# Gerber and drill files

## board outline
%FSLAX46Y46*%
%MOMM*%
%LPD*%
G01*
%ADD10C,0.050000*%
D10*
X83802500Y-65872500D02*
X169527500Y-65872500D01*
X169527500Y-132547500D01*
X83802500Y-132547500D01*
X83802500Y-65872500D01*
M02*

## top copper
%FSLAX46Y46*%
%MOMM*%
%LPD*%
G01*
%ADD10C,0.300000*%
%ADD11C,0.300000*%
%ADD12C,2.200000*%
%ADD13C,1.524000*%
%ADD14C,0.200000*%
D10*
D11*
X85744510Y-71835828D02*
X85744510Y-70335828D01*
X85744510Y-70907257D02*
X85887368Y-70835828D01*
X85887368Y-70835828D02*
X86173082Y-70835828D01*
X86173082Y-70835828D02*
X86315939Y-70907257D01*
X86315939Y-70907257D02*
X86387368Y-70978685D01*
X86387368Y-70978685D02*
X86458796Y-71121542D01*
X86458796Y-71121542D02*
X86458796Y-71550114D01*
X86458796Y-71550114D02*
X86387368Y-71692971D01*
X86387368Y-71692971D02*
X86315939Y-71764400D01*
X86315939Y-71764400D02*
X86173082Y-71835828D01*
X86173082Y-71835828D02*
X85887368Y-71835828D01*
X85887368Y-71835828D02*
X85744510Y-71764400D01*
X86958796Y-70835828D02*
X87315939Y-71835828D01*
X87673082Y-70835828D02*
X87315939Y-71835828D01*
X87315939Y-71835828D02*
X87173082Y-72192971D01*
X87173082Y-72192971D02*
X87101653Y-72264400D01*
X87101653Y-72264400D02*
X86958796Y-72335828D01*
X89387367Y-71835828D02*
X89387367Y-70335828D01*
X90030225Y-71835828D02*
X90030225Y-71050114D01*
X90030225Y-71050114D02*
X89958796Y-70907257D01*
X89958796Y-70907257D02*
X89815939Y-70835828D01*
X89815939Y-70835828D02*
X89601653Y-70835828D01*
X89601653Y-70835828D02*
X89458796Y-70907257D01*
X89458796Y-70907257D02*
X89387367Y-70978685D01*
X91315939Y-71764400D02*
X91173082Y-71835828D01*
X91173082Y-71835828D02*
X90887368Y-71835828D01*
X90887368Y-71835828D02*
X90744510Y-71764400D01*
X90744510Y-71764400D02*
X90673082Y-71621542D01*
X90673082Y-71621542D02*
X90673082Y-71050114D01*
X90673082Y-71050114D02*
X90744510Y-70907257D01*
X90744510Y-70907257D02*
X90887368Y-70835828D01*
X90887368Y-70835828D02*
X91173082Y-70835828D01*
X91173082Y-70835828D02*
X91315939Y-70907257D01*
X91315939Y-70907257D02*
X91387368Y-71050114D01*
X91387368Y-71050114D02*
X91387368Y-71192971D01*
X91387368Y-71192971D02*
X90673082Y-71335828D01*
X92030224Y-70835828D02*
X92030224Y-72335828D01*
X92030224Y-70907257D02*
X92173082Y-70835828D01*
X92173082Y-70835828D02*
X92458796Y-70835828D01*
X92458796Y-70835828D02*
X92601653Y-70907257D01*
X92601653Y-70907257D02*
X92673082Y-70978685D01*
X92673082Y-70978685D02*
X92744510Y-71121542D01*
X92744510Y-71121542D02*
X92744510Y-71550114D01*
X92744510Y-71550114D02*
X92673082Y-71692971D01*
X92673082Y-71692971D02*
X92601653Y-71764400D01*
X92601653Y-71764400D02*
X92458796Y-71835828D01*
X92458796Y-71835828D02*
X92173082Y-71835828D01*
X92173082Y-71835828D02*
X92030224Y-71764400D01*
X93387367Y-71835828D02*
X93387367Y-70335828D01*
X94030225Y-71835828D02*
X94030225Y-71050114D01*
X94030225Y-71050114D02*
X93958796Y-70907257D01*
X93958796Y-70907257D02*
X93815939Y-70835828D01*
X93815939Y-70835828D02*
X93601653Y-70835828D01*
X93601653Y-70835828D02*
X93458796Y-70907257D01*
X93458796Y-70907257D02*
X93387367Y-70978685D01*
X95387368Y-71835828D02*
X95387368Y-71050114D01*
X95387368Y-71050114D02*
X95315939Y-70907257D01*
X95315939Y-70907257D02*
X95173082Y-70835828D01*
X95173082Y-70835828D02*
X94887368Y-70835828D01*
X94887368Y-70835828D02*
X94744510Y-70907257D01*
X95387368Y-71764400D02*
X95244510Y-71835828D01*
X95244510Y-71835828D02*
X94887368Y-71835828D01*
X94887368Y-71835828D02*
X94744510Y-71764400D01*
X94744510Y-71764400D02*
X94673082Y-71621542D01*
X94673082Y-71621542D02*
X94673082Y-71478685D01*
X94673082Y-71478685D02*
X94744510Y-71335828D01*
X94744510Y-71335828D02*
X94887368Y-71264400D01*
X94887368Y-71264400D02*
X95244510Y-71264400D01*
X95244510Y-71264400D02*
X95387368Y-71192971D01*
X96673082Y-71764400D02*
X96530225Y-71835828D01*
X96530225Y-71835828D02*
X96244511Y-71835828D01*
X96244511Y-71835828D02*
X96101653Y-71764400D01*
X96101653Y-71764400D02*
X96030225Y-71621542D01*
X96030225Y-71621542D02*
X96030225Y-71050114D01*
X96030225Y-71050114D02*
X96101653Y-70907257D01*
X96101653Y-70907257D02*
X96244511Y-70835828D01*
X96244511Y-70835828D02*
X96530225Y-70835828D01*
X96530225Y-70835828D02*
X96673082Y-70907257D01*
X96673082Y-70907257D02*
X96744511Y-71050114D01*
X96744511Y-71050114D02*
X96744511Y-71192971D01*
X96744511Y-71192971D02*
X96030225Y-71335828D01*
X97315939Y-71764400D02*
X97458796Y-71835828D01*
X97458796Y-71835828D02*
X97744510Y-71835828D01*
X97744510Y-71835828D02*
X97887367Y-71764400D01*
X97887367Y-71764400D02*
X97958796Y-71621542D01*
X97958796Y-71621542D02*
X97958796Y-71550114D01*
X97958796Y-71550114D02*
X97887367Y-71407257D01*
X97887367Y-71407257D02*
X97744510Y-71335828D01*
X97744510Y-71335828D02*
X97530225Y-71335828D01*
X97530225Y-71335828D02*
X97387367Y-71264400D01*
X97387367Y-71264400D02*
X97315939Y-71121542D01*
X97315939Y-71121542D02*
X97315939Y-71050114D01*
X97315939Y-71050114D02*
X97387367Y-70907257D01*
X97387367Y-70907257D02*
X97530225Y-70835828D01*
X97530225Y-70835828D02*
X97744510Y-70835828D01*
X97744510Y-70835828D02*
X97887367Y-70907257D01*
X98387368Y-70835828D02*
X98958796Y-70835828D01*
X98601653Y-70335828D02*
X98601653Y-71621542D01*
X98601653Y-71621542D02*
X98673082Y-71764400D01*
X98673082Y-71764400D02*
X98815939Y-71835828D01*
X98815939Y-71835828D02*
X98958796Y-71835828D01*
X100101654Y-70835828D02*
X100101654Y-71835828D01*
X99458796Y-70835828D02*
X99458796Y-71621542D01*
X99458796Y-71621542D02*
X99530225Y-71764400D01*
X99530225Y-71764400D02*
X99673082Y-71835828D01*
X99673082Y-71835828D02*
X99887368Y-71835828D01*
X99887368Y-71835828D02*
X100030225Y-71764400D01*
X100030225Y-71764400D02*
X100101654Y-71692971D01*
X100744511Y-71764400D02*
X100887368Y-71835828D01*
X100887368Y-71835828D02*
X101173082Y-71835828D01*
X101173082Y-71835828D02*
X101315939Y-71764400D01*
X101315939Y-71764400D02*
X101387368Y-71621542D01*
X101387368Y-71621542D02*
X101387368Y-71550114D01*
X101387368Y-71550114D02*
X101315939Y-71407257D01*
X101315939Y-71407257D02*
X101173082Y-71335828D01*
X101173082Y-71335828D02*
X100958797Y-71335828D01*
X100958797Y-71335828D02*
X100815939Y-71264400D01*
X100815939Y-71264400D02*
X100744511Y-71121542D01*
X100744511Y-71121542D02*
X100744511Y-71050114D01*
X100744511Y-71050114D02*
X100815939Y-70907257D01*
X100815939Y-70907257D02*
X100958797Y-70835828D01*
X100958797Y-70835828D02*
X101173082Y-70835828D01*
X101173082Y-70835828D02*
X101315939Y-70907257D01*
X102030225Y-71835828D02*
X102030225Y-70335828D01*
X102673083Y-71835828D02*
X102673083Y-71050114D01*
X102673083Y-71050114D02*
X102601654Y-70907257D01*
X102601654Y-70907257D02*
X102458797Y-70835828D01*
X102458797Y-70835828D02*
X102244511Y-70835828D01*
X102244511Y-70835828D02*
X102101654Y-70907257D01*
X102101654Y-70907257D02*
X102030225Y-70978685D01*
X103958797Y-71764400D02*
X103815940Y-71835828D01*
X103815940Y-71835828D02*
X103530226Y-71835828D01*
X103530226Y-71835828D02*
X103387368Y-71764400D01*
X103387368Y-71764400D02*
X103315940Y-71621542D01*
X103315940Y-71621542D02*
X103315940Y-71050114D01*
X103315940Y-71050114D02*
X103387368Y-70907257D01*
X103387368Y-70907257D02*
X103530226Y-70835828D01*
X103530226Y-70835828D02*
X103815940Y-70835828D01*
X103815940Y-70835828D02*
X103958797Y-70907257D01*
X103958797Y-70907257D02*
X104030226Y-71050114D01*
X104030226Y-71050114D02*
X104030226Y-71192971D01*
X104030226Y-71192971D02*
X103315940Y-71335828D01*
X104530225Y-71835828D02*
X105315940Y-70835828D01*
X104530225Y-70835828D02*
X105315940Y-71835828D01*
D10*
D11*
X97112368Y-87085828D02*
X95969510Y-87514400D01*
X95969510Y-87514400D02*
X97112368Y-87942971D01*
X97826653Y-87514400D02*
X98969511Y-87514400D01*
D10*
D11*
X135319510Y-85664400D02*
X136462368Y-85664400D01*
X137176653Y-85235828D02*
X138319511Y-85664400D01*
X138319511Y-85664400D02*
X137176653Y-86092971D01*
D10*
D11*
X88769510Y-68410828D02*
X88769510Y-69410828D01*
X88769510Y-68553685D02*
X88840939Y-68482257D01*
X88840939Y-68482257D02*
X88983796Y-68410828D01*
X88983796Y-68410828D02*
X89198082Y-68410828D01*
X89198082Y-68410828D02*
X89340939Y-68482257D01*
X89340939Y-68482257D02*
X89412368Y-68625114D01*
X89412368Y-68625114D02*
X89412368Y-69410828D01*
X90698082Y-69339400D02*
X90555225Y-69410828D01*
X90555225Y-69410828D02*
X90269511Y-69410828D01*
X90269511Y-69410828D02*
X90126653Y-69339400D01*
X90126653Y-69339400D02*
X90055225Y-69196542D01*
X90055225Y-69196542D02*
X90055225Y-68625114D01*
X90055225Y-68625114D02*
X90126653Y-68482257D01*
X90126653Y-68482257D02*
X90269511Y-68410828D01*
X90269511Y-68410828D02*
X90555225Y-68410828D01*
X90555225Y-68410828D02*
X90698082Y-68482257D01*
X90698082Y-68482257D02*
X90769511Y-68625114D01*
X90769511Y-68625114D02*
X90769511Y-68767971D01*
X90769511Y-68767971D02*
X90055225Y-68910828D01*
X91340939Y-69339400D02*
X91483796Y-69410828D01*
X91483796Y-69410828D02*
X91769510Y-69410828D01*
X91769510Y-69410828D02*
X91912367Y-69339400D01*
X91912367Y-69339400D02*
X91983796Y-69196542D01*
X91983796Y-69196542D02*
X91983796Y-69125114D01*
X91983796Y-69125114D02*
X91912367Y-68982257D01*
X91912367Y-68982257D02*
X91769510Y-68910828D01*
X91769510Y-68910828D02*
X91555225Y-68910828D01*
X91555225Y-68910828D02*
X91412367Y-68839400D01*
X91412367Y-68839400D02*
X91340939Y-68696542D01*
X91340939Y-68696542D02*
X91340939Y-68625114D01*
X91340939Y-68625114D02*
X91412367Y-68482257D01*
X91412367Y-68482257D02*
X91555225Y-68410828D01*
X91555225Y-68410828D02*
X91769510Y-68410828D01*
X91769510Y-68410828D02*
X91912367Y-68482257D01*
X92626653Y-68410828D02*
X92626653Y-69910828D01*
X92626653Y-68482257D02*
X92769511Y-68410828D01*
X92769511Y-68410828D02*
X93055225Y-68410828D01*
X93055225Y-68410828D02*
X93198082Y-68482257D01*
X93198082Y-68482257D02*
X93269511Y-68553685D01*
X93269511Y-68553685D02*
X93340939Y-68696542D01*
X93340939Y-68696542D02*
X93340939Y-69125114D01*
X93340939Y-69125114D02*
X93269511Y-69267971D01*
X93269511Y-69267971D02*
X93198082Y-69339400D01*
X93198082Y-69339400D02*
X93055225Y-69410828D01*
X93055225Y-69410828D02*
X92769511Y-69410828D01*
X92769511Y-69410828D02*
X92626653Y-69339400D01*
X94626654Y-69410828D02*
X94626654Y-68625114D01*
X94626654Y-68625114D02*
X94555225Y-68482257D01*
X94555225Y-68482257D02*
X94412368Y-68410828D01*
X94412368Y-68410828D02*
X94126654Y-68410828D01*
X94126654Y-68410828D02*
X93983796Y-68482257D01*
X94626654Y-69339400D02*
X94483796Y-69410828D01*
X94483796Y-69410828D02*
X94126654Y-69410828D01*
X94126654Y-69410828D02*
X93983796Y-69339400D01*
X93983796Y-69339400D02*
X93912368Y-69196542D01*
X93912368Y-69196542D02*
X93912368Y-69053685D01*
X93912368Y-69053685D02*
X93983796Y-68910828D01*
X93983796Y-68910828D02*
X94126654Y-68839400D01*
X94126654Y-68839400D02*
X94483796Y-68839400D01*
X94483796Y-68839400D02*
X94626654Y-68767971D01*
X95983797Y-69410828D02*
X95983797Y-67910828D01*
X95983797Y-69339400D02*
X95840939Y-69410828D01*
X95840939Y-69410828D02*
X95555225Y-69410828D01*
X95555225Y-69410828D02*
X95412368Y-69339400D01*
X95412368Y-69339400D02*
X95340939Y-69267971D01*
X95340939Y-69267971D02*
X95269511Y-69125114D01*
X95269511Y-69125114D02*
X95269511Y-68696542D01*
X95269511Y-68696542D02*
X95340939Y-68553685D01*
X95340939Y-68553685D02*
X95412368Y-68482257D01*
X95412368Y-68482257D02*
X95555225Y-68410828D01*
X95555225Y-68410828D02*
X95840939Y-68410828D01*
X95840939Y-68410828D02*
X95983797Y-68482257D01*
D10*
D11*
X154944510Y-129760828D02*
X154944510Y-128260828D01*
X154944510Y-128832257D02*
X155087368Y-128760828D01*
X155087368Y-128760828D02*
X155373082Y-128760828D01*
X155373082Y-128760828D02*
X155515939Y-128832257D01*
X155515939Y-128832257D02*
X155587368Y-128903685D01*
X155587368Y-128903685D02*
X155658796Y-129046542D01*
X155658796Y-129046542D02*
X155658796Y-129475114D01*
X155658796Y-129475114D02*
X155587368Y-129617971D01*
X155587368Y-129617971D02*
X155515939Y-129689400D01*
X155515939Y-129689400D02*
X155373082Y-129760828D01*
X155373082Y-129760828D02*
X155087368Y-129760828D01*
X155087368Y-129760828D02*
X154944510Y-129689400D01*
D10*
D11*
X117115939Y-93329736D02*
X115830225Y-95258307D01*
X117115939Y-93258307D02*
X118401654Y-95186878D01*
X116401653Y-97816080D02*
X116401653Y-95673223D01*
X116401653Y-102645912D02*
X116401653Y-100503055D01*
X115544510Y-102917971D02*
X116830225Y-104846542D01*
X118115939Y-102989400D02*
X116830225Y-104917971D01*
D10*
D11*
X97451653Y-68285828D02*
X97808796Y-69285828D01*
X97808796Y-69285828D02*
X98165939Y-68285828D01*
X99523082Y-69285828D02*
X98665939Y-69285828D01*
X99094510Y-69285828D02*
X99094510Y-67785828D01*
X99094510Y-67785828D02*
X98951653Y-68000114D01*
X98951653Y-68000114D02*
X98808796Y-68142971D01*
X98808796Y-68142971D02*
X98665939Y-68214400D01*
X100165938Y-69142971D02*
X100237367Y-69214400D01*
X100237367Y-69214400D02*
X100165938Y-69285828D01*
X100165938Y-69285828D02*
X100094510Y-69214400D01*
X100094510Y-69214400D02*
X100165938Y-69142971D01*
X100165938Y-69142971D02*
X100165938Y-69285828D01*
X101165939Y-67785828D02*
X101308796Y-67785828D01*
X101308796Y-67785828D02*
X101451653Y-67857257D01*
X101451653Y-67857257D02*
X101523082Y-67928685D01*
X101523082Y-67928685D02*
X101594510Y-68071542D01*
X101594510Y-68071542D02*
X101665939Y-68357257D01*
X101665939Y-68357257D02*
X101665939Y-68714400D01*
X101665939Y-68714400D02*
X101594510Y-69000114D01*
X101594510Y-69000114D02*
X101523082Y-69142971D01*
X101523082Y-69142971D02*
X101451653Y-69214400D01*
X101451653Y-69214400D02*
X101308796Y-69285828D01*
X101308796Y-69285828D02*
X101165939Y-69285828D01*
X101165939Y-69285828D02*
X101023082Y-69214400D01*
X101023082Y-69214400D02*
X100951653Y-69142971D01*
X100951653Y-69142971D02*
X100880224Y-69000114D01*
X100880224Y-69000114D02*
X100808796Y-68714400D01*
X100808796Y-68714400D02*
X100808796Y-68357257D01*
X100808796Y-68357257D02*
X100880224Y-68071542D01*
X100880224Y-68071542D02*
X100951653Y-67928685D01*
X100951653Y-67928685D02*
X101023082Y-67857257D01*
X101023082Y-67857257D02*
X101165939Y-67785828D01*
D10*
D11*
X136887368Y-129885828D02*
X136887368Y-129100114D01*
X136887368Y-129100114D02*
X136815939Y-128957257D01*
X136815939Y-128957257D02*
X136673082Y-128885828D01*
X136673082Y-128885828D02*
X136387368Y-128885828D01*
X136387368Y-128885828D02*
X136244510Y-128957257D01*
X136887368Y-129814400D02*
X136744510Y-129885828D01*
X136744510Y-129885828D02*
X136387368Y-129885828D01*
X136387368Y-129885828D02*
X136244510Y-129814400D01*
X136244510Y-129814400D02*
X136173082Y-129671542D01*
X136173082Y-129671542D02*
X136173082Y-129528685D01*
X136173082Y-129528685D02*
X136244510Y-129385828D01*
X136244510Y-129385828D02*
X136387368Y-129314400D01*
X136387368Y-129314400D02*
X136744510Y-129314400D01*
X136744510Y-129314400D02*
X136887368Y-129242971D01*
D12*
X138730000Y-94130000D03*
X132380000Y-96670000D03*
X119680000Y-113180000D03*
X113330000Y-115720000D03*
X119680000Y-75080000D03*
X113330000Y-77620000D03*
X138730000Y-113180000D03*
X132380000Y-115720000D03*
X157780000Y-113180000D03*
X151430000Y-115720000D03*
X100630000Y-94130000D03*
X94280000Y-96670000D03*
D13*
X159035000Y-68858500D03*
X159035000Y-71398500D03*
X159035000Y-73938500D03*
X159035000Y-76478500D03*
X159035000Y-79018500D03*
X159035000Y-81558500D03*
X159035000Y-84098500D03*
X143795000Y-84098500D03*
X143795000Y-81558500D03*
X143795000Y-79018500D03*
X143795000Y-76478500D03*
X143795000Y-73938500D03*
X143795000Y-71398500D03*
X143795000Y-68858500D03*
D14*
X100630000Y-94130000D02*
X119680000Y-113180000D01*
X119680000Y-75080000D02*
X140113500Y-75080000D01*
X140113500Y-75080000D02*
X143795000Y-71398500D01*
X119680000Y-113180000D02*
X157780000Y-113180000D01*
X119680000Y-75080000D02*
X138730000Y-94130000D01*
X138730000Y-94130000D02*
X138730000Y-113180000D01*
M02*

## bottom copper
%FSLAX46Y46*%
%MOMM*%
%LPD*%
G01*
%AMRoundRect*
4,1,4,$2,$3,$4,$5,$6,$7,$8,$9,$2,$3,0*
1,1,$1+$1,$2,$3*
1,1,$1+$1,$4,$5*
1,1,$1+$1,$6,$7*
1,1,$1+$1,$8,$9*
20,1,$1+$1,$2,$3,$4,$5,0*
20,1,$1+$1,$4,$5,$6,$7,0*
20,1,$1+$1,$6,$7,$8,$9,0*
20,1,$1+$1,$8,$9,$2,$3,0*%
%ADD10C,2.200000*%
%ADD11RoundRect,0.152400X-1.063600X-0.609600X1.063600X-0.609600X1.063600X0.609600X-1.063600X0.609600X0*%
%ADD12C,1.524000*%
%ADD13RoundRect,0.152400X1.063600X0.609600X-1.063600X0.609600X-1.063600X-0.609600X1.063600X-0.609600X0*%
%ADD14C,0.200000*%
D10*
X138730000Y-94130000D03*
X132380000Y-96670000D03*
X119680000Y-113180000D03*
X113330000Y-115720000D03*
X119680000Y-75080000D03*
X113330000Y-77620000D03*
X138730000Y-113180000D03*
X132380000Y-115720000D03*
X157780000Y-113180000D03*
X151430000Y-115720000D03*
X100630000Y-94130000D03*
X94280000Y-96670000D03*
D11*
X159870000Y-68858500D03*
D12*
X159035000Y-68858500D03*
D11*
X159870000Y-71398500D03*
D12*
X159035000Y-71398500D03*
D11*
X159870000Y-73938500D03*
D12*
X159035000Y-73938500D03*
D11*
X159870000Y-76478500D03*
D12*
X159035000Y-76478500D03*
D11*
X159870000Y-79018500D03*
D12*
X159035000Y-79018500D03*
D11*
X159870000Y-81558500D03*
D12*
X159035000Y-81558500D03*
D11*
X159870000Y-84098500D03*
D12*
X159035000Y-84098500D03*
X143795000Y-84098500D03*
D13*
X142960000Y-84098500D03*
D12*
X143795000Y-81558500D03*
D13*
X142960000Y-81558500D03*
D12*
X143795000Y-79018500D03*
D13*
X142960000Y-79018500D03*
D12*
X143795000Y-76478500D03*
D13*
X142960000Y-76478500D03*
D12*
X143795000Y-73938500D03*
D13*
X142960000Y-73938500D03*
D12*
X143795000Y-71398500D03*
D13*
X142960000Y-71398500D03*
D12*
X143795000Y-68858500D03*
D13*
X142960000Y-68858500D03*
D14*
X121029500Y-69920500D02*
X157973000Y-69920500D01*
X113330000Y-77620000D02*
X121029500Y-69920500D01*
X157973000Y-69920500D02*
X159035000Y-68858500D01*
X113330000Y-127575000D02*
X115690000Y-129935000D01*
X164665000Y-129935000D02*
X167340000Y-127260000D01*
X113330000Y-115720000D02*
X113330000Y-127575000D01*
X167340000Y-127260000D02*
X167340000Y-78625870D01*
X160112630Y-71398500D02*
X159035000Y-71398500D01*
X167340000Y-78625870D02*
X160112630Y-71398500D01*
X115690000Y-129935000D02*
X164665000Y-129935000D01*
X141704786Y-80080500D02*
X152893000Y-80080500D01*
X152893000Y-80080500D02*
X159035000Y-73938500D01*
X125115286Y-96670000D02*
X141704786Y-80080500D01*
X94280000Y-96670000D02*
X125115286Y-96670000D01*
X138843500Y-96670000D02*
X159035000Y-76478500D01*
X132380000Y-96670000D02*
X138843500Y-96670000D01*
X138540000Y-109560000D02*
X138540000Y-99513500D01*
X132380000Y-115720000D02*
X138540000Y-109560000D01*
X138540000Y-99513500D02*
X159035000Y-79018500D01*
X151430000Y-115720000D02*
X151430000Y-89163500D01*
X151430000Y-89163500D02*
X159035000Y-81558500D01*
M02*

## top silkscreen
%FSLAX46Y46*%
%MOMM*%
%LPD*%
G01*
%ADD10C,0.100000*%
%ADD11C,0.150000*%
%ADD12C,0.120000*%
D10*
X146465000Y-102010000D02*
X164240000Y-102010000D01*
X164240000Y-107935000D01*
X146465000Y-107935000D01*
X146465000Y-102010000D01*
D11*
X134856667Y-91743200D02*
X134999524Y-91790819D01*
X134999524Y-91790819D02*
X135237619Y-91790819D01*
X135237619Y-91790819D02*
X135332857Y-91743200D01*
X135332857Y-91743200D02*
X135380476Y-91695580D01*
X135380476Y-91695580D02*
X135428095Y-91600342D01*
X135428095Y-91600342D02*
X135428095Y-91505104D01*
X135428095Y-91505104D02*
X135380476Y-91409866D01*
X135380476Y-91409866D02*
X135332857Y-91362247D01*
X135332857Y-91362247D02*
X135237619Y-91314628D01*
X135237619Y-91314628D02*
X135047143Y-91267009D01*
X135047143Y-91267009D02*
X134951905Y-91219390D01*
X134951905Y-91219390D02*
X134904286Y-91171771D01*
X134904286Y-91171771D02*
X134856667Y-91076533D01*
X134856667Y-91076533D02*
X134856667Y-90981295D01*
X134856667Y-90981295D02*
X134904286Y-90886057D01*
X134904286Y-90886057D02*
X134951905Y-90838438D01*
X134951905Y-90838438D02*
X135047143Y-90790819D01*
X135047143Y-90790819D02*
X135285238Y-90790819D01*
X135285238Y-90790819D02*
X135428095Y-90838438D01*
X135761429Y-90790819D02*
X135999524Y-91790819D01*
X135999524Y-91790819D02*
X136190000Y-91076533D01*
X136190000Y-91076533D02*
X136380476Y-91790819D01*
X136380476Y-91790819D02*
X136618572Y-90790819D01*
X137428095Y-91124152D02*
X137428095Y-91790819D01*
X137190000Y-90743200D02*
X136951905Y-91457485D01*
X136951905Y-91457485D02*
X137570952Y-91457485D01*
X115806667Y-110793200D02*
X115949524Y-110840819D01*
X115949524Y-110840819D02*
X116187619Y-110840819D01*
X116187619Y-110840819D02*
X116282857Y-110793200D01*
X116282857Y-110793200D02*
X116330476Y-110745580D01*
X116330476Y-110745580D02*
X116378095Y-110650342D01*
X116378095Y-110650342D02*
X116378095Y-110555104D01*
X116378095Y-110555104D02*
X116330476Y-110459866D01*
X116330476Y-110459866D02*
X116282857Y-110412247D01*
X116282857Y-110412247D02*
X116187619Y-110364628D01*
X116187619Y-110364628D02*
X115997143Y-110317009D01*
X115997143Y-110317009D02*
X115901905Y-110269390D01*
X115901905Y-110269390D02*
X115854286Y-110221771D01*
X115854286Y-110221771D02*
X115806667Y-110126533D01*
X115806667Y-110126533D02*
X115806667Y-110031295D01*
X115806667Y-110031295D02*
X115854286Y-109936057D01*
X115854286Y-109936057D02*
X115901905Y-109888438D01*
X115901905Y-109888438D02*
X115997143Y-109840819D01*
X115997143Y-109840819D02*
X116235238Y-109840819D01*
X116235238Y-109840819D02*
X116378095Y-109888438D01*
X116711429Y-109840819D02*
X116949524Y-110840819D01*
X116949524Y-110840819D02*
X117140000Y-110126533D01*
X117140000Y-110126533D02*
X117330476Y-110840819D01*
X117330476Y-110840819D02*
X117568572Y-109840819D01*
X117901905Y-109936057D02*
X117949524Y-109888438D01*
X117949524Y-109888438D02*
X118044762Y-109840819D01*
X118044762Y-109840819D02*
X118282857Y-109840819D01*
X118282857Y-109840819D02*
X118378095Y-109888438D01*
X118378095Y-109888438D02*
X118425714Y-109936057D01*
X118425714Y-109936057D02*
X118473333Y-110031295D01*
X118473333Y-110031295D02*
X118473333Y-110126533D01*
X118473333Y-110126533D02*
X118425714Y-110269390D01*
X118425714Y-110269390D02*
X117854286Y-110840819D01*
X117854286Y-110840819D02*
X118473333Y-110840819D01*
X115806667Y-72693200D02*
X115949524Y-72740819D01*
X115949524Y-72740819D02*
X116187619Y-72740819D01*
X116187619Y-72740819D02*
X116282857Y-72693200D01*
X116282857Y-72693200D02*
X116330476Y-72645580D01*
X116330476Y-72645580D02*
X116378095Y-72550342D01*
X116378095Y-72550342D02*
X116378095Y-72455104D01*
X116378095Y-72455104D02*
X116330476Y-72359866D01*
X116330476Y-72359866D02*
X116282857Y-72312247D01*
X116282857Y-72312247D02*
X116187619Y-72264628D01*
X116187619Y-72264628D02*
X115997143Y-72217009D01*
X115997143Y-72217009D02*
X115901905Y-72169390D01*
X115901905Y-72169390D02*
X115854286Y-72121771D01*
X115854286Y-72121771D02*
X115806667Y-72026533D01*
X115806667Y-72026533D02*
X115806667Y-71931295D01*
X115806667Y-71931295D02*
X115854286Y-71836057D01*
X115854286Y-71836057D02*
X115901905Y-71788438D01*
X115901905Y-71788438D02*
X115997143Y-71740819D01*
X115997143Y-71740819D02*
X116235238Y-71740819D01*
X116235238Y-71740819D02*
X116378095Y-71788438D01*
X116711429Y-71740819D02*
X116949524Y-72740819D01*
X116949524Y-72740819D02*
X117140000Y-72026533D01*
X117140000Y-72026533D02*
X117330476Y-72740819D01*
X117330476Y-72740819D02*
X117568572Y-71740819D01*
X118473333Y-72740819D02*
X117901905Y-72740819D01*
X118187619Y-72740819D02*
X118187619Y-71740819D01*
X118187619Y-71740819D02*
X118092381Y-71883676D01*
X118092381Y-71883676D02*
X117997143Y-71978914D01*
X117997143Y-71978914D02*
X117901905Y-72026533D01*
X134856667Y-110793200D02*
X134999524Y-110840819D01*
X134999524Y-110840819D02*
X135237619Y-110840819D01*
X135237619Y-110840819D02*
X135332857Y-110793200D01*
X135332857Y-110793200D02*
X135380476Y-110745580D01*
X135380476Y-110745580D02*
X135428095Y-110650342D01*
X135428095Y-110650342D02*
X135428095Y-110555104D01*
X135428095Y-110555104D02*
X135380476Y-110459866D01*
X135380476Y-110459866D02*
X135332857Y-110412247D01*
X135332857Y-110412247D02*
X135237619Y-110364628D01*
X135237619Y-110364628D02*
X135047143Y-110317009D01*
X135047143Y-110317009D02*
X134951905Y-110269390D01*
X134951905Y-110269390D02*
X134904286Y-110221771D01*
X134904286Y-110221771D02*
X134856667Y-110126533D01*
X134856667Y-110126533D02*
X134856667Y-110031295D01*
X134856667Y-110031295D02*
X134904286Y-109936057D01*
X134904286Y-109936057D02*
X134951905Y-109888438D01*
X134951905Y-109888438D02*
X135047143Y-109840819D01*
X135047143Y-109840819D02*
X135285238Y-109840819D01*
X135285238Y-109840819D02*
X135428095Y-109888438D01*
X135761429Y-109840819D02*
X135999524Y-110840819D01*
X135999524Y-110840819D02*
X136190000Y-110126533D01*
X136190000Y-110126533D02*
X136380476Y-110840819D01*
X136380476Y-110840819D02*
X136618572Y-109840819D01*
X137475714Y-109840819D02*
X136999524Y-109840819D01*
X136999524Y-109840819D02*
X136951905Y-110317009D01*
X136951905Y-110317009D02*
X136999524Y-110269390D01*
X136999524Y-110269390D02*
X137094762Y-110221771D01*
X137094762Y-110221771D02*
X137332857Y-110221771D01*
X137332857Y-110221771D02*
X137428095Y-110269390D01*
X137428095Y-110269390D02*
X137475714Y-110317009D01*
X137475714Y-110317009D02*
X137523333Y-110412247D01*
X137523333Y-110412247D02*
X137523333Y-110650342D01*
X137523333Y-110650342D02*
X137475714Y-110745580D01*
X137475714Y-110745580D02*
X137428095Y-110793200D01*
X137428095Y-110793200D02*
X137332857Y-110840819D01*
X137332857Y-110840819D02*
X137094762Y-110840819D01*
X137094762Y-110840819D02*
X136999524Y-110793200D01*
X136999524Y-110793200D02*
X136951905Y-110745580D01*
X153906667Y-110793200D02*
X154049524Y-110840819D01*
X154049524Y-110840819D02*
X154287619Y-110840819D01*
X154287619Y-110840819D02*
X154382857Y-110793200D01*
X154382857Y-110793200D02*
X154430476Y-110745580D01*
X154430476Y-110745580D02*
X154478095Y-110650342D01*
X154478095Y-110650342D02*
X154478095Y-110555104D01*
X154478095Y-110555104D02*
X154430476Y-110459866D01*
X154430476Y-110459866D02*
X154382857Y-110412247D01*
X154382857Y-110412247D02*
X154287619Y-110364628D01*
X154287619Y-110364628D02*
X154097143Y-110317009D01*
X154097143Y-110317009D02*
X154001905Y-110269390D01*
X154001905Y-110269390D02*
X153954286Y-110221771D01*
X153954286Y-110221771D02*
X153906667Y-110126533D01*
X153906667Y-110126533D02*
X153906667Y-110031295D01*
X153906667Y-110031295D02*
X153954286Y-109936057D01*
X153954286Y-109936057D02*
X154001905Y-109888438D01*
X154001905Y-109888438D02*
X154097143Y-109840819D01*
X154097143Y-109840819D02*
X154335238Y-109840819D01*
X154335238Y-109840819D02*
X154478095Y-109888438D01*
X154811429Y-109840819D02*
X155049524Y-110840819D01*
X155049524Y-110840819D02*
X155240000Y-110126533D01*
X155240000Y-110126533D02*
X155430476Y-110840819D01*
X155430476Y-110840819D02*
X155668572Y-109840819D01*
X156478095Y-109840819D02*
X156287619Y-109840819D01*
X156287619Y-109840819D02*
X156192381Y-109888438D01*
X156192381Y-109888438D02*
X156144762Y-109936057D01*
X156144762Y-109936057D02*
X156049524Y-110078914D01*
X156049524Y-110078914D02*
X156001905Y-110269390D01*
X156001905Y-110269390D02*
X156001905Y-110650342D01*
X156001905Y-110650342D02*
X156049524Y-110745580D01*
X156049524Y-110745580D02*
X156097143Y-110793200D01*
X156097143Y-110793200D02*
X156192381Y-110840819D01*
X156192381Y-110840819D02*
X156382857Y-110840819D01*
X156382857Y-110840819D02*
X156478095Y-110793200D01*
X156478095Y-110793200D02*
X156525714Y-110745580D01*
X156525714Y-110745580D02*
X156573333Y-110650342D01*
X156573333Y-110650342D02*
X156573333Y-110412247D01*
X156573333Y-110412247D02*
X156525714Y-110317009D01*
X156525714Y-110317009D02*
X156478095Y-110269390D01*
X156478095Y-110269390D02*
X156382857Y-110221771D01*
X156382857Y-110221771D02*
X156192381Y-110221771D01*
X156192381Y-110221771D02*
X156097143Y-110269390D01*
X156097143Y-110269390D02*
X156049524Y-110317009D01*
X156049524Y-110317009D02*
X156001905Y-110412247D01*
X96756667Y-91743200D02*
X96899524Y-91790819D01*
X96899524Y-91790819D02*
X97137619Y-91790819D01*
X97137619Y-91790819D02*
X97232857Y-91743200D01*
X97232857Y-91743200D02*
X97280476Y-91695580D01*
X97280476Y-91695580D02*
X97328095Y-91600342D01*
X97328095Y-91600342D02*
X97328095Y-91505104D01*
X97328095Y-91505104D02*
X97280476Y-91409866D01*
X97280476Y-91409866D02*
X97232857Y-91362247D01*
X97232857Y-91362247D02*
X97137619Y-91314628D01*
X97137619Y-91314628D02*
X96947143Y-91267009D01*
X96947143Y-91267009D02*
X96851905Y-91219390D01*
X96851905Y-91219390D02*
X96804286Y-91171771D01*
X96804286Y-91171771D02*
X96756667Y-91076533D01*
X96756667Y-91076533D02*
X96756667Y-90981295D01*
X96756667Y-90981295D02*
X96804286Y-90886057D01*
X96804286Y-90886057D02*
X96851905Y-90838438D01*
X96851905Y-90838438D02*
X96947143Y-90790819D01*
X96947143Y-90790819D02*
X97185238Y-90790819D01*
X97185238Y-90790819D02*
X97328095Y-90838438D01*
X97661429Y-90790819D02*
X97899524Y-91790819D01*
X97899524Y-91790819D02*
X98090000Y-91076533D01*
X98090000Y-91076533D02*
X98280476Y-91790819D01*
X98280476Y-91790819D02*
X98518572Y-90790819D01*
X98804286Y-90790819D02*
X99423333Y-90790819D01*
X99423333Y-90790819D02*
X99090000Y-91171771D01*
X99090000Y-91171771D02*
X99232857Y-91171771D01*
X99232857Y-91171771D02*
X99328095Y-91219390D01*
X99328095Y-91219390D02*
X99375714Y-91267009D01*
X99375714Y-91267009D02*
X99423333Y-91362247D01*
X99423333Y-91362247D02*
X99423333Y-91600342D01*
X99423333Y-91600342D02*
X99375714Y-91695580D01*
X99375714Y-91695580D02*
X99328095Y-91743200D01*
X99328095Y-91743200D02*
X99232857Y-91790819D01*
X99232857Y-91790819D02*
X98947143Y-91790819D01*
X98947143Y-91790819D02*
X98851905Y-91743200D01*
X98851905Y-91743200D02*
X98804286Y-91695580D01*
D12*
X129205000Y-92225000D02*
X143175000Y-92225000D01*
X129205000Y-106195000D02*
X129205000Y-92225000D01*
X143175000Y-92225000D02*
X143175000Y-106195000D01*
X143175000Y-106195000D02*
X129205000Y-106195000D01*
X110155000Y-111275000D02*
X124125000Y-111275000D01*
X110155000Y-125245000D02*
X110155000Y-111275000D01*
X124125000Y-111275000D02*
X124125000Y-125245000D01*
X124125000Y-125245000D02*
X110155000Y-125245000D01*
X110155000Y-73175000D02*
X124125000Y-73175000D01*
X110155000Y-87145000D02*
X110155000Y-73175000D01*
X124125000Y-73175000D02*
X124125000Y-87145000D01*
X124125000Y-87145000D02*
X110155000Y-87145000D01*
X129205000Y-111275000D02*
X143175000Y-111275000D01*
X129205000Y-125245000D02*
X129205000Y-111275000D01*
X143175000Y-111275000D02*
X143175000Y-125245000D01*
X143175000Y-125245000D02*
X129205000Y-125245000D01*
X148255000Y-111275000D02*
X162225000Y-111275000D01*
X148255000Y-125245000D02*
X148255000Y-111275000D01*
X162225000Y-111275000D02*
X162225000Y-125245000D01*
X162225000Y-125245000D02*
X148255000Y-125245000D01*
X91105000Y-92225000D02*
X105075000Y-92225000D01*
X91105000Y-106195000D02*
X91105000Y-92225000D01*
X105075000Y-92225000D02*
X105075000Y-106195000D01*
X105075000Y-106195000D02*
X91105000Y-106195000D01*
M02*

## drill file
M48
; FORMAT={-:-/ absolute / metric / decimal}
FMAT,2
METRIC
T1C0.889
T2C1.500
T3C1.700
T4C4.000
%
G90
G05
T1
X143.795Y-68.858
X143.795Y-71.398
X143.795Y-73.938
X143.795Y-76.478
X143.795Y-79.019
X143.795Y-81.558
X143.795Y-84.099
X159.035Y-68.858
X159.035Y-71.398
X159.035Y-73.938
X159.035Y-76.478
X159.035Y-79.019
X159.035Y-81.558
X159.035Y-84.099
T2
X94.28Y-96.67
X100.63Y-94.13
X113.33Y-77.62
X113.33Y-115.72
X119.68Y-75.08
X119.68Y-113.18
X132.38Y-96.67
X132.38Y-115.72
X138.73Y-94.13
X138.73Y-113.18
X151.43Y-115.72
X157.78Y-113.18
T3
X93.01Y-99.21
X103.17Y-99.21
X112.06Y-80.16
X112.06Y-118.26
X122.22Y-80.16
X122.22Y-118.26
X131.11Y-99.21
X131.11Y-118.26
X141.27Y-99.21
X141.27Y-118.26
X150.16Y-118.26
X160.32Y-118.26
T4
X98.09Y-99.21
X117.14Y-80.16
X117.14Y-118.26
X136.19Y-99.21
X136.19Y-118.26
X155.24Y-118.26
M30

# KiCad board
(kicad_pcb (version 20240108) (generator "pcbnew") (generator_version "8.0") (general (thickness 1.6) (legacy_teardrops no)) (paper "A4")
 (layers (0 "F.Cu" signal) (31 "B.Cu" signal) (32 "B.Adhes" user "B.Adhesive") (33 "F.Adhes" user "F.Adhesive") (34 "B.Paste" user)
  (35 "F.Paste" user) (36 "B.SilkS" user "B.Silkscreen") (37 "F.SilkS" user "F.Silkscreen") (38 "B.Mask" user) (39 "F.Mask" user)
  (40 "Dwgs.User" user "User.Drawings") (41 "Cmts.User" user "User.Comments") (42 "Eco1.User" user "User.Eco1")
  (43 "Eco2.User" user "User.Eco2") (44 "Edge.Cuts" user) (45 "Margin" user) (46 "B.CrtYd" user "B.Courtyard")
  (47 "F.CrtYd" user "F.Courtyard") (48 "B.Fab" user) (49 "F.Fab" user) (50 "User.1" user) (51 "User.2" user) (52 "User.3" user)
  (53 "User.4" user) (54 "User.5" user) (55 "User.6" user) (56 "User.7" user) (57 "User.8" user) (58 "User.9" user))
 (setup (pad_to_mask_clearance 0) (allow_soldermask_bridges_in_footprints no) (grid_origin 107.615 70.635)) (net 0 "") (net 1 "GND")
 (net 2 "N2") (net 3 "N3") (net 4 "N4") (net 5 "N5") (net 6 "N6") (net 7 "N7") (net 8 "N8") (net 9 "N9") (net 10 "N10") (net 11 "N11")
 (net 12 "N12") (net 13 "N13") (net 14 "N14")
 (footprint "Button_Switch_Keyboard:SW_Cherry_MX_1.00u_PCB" (layer "F.Cu") (at 138.73 94.13)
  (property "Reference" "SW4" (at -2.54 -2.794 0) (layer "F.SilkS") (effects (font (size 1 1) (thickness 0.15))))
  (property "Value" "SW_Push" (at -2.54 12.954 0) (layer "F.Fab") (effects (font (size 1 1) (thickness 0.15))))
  (fp_line (start -9.525 -1.905) (end 4.445 -1.905) (stroke (width 0.12) (type solid)) (layer "F.SilkS"))
  (fp_line (start -9.525 12.065) (end -9.525 -1.905) (stroke (width 0.12) (type solid)) (layer "F.SilkS"))
  (fp_line (start 4.445 -1.905) (end 4.445 12.065) (stroke (width 0.12) (type solid)) (layer "F.SilkS"))
  (fp_line (start 4.445 12.065) (end -9.525 12.065) (stroke (width 0.12) (type solid)) (layer "F.SilkS"))
  (pad "" np_thru_hole circle (at -7.62 5.08) (size 1.7 1.7) (drill 1.7) (layers "*.Cu" "*.Mask"))
  (pad "" np_thru_hole circle (at -2.54 5.08) (size 4 4) (drill 4) (layers "*.Cu" "*.Mask"))
  (pad "" np_thru_hole circle (at 2.54 5.08) (size 1.7 1.7) (drill 1.7) (layers "*.Cu" "*.Mask"))
  (pad "1" thru_hole circle (at 0 0) (size 2.2 2.2) (drill 1.5) (layers "*.Cu" "*.Mask") (remove_unused_layers no) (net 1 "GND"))
  (pad "2" thru_hole circle (at -6.35 2.54) (size 2.2 2.2) (drill 1.5) (layers "*.Cu" "*.Mask") (remove_unused_layers no) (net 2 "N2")))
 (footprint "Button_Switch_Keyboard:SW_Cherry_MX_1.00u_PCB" (layer "F.Cu") (at 119.68 113.18)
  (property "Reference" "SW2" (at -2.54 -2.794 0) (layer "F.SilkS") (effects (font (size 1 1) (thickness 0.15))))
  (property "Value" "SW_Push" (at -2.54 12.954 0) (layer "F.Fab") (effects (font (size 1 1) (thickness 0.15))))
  (fp_line (start -9.525 -1.905) (end 4.445 -1.905) (stroke (width 0.12) (type solid)) (layer "F.SilkS"))
  (fp_line (start -9.525 12.065) (end -9.525 -1.905) (stroke (width 0.12) (type solid)) (layer "F.SilkS"))
  (fp_line (start 4.445 -1.905) (end 4.445 12.065) (stroke (width 0.12) (type solid)) (layer "F.SilkS"))
  (fp_line (start 4.445 12.065) (end -9.525 12.065) (stroke (width 0.12) (type solid)) (layer "F.SilkS"))
  (pad "" np_thru_hole circle (at -7.62 5.08) (size 1.7 1.7) (drill 1.7) (layers "*.Cu" "*.Mask"))
  (pad "" np_thru_hole circle (at -2.54 5.08) (size 4 4) (drill 4) (layers "F&B.Cu" "*.Mask"))
  (pad "" np_thru_hole circle (at 2.54 5.08) (size 1.7 1.7) (drill 1.7) (layers "*.Cu" "*.Mask"))
  (pad "1" thru_hole circle (at 0 0) (size 2.2 2.2) (drill 1.5) (layers "*.Cu" "*.Mask") (remove_unused_layers no) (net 1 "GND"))
  (pad "2" thru_hole circle (at -6.35 2.54) (size 2.2 2.2) (drill 1.5) (layers "*.Cu" "*.Mask") (remove_unused_layers no) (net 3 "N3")))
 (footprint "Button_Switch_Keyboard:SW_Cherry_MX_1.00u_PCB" (layer "F.Cu") (at 119.68 75.08)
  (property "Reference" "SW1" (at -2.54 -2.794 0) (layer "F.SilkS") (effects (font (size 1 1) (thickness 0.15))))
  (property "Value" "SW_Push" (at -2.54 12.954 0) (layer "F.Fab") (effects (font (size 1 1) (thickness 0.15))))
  (fp_line (start -9.525 -1.905) (end 4.445 -1.905) (stroke (width 0.12) (type solid)) (layer "F.SilkS"))
  (fp_line (start -9.525 12.065) (end -9.525 -1.905) (stroke (width 0.12) (type solid)) (layer "F.SilkS"))
  (fp_line (start 4.445 -1.905) (end 4.445 12.065) (stroke (width 0.12) (type solid)) (layer "F.SilkS"))
  (fp_line (start 4.445 12.065) (end -9.525 12.065) (stroke (width 0.12) (type solid)) (layer "F.SilkS"))
  (pad "" np_thru_hole circle (at -7.62 5.08) (size 1.7 1.7) (drill 1.7) (layers "*.Cu" "*.Mask"))
  (pad "" np_thru_hole circle (at -2.54 5.08) (size 4 4) (drill 4) (layers "*.Cu" "*.Mask"))
  (pad "" np_thru_hole circle (at 2.54 5.08) (size 1.7 1.7) (drill 1.7) (layers "*.Cu" "*.Mask"))
  (pad "1" thru_hole circle (at 0 0) (size 2.2 2.2) (drill 1.5) (layers "*.Cu" "*.Mask") (remove_unused_layers no) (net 1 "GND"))
  (pad "2" thru_hole circle (at -6.35 2.54) (size 2.2 2.2) (drill 1.5) (layers "*.Cu" "*.Mask") (remove_unused_layers no) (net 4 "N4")))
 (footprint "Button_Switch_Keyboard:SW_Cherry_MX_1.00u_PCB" (layer "F.Cu") (at 138.73 113.18)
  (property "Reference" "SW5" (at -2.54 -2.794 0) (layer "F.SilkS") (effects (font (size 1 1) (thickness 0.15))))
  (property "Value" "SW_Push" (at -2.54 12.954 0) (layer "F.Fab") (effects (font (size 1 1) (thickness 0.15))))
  (fp_line (start -9.525 -1.905) (end 4.445 -1.905) (stroke (width 0.12) (type solid)) (layer "F.SilkS"))
  (fp_line (start -9.525 12.065) (end -9.525 -1.905) (stroke (width 0.12) (type solid)) (layer "F.SilkS"))
  (fp_line (start 4.445 -1.905) (end 4.445 12.065) (stroke (width 0.12) (type solid)) (layer "F.SilkS"))
  (fp_line (start 4.445 12.065) (end -9.525 12.065) (stroke (width 0.12) (type solid)) (layer "F.SilkS"))
  (pad "" np_thru_hole circle (at -7.62 5.08) (size 1.7 1.7) (drill 1.7) (layers "*.Cu" "*.Mask"))
  (pad "" np_thru_hole circle (at -2.54 5.08) (size 4 4) (drill 4) (layers "F&B.Cu" "*.Mask"))
  (pad "" np_thru_hole circle (at 2.54 5.08) (size 1.7 1.7) (drill 1.7) (layers "*.Cu" "*.Mask"))
  (pad "1" thru_hole circle (at 0 0) (size 2.2 2.2) (drill 1.5) (layers "*.Cu" "*.Mask") (remove_unused_layers no) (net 1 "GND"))
  (pad "2" thru_hole circle (at -6.35 2.54) (size 2.2 2.2) (drill 1.5) (layers "*.Cu" "*.Mask") (remove_unused_layers no) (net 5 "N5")))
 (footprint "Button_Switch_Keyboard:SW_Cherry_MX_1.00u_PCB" (layer "F.Cu") (at 157.78 113.18)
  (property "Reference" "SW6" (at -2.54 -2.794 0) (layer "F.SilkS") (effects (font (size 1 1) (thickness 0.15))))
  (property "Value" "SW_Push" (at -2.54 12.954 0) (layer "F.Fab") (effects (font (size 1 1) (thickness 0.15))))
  (fp_line (start -9.525 -1.905) (end 4.445 -1.905) (stroke (width 0.12) (type solid)) (layer "F.SilkS"))
  (fp_line (start -9.525 12.065) (end -9.525 -1.905) (stroke (width 0.12) (type solid)) (layer "F.SilkS"))
  (fp_line (start 4.445 -1.905) (end 4.445 12.065) (stroke (width 0.12) (type solid)) (layer "F.SilkS"))
  (fp_line (start 4.445 12.065) (end -9.525 12.065) (stroke (width 0.12) (type solid)) (layer "F.SilkS"))
  (pad "" np_thru_hole circle (at -7.62 5.08) (size 1.7 1.7) (drill 1.7) (layers "*.Cu" "*.Mask"))
  (pad "" np_thru_hole circle (at -2.54 5.08) (size 4 4) (drill 4) (layers "*.Cu" "*.Mask"))
  (pad "" np_thru_hole circle (at 2.54 5.08) (size 1.7 1.7) (drill 1.7) (layers "*.Cu" "*.Mask"))
  (pad "1" thru_hole circle (at 0 0) (size 2.2 2.2) (drill 1.5) (layers "*.Cu" "*.Mask") (remove_unused_layers no) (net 1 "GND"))
  (pad "2" thru_hole circle (at -6.35 2.54) (size 2.2 2.2) (drill 1.5) (layers "*.Cu" "*.Mask") (remove_unused_layers no) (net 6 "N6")))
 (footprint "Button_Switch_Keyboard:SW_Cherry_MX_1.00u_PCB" (layer "F.Cu") (at 100.63 94.13)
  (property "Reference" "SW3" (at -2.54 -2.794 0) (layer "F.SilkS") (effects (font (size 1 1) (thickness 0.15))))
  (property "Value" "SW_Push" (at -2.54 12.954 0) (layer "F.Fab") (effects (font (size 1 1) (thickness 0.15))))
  (fp_line (start -9.525 -1.905) (end 4.445 -1.905) (stroke (width 0.12) (type solid)) (layer "F.SilkS"))
  (fp_line (start -9.525 12.065) (end -9.525 -1.905) (stroke (width 0.12) (type solid)) (layer "F.SilkS"))
  (fp_line (start 4.445 -1.905) (end 4.445 12.065) (stroke (width 0.12) (type solid)) (layer "F.SilkS"))
  (fp_line (start 4.445 12.065) (end -9.525 12.065) (stroke (width 0.12) (type solid)) (layer "F.SilkS"))
  (pad "" np_thru_hole circle (at -7.62 5.08) (size 1.7 1.7) (drill 1.7) (layers "*.Cu" "*.Mask"))
  (pad "" np_thru_hole circle (at -2.54 5.08) (size 4 4) (drill 4) (layers "F&B.Cu" "*.Mask"))
  (pad "" np_thru_hole circle (at 2.54 5.08) (size 1.7 1.7) (drill 1.7) (layers "*.Cu" "*.Mask"))
  (pad "1" thru_hole circle (at 0 0) (size 2.2 2.2) (drill 1.5) (layers "*.Cu" "*.Mask") (remove_unused_layers no) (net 1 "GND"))
  (pad "2" thru_hole circle (at -6.35 2.54) (size 2.2 2.2) (drill 1.5) (layers "*.Cu" "*.Mask") (remove_unused_layers no) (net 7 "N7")))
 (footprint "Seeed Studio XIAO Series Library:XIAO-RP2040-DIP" (layer "B.Cu") (at 151.415 76.4785 180)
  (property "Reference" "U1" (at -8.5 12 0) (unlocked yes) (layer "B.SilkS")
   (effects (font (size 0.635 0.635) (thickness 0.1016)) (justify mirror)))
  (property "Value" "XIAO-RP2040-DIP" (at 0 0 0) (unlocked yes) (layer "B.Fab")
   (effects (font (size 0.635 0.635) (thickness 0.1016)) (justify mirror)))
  (pad "1" smd roundrect (at -8.455 7.62) (size 2.432 1.524) (layers "B.Cu" "B.Mask") (roundrect_rratio 0.1) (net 4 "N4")
   (thermal_bridge_angle 45))
  (pad "1" thru_hole circle (at -7.62 7.62) (size 1.524 1.524) (drill 0.889) (layers "*.Cu" "*.Mask") (remove_unused_layers no) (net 4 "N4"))
  (pad "2" smd roundrect (at -8.455 5.08) (size 2.432 1.524) (layers "B.Cu" "B.Mask") (roundrect_rratio 0.1) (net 3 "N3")
   (thermal_bridge_angle 45))
  (pad "2" thru_hole circle (at -7.62 5.08) (size 1.524 1.524) (drill 0.889) (layers "*.Cu" "*.Mask") (remove_unused_layers no) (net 3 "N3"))
  (pad "3" smd roundrect (at -8.455 2.54) (size 2.432 1.524) (layers "B.Cu" "B.Mask") (roundrect_rratio 0.1) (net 7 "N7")
   (thermal_bridge_angle 45))
  (pad "3" thru_hole circle (at -7.62 2.54) (size 1.524 1.524) (drill 0.889) (layers "*.Cu" "*.Mask") (remove_unused_layers no) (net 7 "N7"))
  (pad "4" smd roundrect (at -8.455 0) (size 2.432 1.524) (layers "B.Cu" "B.Mask") (roundrect_rratio 0.1) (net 2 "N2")
   (thermal_bridge_angle 45))
  (pad "4" thru_hole circle (at -7.62 0) (size 1.524 1.524) (drill 0.889) (layers "*.Cu" "*.Mask") (remove_unused_layers no) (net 2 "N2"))
  (pad "5" smd roundrect (at -8.455 -2.54) (size 2.432 1.524) (layers "B.Cu" "B.Mask") (roundrect_rratio 0.1) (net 5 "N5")
   (thermal_bridge_angle 45))
  (pad "5" thru_hole circle (at -7.62 -2.54) (size 1.524 1.524) (drill 0.889) (layers "*.Cu" "*.Mask") (remove_unused_layers no)
   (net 5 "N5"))
  (pad "6" smd roundrect (at -8.455 -5.08) (size 2.432 1.524) (layers "B.Cu" "B.Mask") (roundrect_rratio 0.1) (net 6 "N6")
   (thermal_bridge_angle 45))
  (pad "6" thru_hole circle (at -7.62 -5.08) (size 1.524 1.524) (drill 0.889) (layers "*.Cu" "*.Mask") (remove_unused_layers no)
   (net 6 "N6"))
  (pad "7" smd roundrect (at -8.455 -7.62) (size 2.432 1.524) (layers "B.Cu" "B.Mask") (roundrect_rratio 0.1) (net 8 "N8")
   (thermal_bridge_angle 45))
  (pad "7" thru_hole circle (at -7.62 -7.62) (size 1.524 1.524) (drill 0.889) (layers "*.Cu" "*.Mask") (remove_unused_layers no)
   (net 8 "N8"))
  (pad "8" thru_hole circle (at 7.62 -7.62 180) (size 1.524 1.524) (drill 0.889) (layers "*.Cu" "*.Mask") (remove_unused_layers no)
   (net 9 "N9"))
  (pad "8" smd roundrect (at 8.455 -7.62 180) (size 2.432 1.524) (layers "B.Cu" "B.Mask") (roundrect_rratio 0.1) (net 9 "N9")
   (thermal_bridge_angle 45))
  (pad "9" thru_hole circle (at 7.62 -5.08 180) (size 1.524 1.524) (drill 0.889) (layers "*.Cu" "*.Mask") (remove_unused_layers no)
   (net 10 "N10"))
  (pad "9" smd roundrect (at 8.455 -5.08 180) (size 2.432 1.524) (layers "B.Cu" "B.Mask") (roundrect_rratio 0.1) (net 10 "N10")
   (thermal_bridge_angle 45))
  (pad "10" thru_hole circle (at 7.62 -2.54 180) (size 1.524 1.524) (drill 0.889) (layers "*.Cu" "*.Mask") (remove_unused_layers no)
   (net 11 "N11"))
  (pad "10" smd roundrect (at 8.455 -2.54 180) (size 2.432 1.524) (layers "B.Cu" "B.Mask") (roundrect_rratio 0.1) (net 11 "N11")
   (thermal_bridge_angle 45))
  (pad "11" thru_hole circle (at 7.62 0 180) (size 1.524 1.524) (drill 0.889) (layers "*.Cu" "*.Mask") (remove_unused_layers no)
   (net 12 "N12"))
  (pad "11" smd roundrect (at 8.455 0 180) (size 2.432 1.524) (layers "B.Cu" "B.Mask") (roundrect_rratio 0.1) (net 12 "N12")
   (thermal_bridge_angle 45))
  (pad "12" thru_hole circle (at 7.62 2.54 180) (size 1.524 1.524) (drill 0.889) (layers "*.Cu" "*.Mask") (remove_unused_layers no)
   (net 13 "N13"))
  (pad "12" smd roundrect (at 8.455 2.54 180) (size 2.432 1.524) (layers "B.Cu" "B.Mask") (roundrect_rratio 0.1) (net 13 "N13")
   (thermal_bridge_angle 45))
  (pad "13" thru_hole circle (at 7.62 5.08 180) (size 1.524 1.524) (drill 0.889) (layers "*.Cu" "*.Mask") (remove_unused_layers no)
   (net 1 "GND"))
  (pad "13" smd roundrect (at 8.455 5.08 180) (size 2.432 1.524) (layers "B.Cu" "B.Mask") (roundrect_rratio 0.1) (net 1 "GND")
   (thermal_bridge_angle 45))
  (pad "14" thru_hole circle (at 7.62 7.62 180) (size 1.524 1.524) (drill 0.889) (layers "*.Cu" "*.Mask") (remove_unused_layers no)
   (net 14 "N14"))
  (pad "14" smd roundrect (at 8.455 7.62 180) (size 2.432 1.524) (layers "B.Cu" "B.Mask") (roundrect_rratio 0.1) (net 14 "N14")
   (thermal_bridge_angle 45)))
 (gr_rect (start 146.465 102.01) (end 164.24 107.935) (stroke (width 0.1) (type default)) (fill none) (layer "F.SilkS"))
 (gr_rect (start 83.8025 65.8725) (end 169.5275 132.5475) (stroke (width 0.05) (type default)) (fill none) (layer "Edge.Cuts"))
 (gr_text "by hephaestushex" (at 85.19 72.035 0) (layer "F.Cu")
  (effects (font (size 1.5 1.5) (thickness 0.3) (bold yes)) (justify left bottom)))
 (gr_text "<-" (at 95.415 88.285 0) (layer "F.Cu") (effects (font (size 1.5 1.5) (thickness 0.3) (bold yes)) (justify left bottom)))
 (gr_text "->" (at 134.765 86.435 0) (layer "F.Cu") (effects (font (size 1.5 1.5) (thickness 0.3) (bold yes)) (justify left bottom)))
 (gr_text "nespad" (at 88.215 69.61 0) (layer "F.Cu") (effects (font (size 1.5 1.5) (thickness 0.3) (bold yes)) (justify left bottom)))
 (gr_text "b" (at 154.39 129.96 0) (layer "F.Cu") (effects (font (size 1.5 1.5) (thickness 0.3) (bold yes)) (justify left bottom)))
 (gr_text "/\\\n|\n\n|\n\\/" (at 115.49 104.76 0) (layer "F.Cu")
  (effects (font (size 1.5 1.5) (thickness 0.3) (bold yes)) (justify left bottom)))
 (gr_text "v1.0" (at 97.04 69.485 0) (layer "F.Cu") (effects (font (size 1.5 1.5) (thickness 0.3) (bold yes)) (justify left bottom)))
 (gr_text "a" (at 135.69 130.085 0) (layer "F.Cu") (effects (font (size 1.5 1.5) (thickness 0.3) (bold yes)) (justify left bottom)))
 (segment (start 121.0295 69.9205) (end 157.973 69.9205) (width 0.2) (layer "B.Cu") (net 4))
 (segment (start 113.33 77.62) (end 121.0295 69.9205) (width 0.2) (layer "B.Cu") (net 4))
 (segment (start 157.973 69.9205) (end 159.035 68.8585) (width 0.2) (layer "B.Cu") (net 4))
 (segment (start 100.63 94.13) (end 119.68 113.18) (width 0.2) (layer "F.Cu") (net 1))
 (segment (start 119.68 75.08) (end 140.1135 75.08) (width 0.2) (layer "F.Cu") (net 1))
 (segment (start 140.1135 75.08) (end 143.795 71.3985) (width 0.2) (layer "F.Cu") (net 1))
 (segment (start 119.68 113.18) (end 157.78 113.18) (width 0.2) (layer "F.Cu") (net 1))
 (segment (start 119.68 75.08) (end 138.73 94.13) (width 0.2) (layer "F.Cu") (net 1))
 (segment (start 138.73 94.13) (end 138.73 113.18) (width 0.2) (layer "F.Cu") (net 1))
 (segment (start 113.33 127.575) (end 115.69 129.935) (width 0.2) (layer "B.Cu") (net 3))
 (segment (start 164.665 129.935) (end 167.34 127.26) (width 0.2) (layer "B.Cu") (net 3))
 (segment (start 113.33 115.72) (end 113.33 127.575) (width 0.2) (layer "B.Cu") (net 3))
 (segment (start 167.34 127.26) (end 167.34 78.62587) (width 0.2) (layer "B.Cu") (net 3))
 (segment (start 160.11263 71.3985) (end 159.035 71.3985) (width 0.2) (layer "B.Cu") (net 3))
 (segment (start 167.34 78.62587) (end 160.11263 71.3985) (width 0.2) (layer "B.Cu") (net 3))
 (segment (start 115.69 129.935) (end 164.665 129.935) (width 0.2) (layer "B.Cu") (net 3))
 (segment (start 141.704786 80.0805) (end 152.893 80.0805) (width 0.2) (layer "B.Cu") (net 7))
 (segment (start 152.893 80.0805) (end 159.035 73.9385) (width 0.2) (layer "B.Cu") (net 7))
 (segment (start 125.115286 96.67) (end 141.704786 80.0805) (width 0.2) (layer "B.Cu") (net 7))
 (segment (start 94.28 96.67) (end 125.115286 96.67) (width 0.2) (layer "B.Cu") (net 7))
 (segment (start 138.8435 96.67) (end 159.035 76.4785) (width 0.2) (layer "B.Cu") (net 2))
 (segment (start 132.38 96.67) (end 138.8435 96.67) (width 0.2) (layer "B.Cu") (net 2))
 (segment (start 138.54 109.56) (end 138.54 99.5135) (width 0.2) (layer "B.Cu") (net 5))
 (segment (start 132.38 115.72) (end 138.54 109.56) (width 0.2) (layer "B.Cu") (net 5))
 (segment (start 138.54 99.5135) (end 159.035 79.0185) (width 0.2) (layer "B.Cu") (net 5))
 (segment (start 151.43 115.72) (end 151.43 89.1635) (width 0.2) (layer "B.Cu") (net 6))
 (segment (start 151.43 89.1635) (end 159.035 81.5585) (width 0.2) (layer "B.Cu") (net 6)))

